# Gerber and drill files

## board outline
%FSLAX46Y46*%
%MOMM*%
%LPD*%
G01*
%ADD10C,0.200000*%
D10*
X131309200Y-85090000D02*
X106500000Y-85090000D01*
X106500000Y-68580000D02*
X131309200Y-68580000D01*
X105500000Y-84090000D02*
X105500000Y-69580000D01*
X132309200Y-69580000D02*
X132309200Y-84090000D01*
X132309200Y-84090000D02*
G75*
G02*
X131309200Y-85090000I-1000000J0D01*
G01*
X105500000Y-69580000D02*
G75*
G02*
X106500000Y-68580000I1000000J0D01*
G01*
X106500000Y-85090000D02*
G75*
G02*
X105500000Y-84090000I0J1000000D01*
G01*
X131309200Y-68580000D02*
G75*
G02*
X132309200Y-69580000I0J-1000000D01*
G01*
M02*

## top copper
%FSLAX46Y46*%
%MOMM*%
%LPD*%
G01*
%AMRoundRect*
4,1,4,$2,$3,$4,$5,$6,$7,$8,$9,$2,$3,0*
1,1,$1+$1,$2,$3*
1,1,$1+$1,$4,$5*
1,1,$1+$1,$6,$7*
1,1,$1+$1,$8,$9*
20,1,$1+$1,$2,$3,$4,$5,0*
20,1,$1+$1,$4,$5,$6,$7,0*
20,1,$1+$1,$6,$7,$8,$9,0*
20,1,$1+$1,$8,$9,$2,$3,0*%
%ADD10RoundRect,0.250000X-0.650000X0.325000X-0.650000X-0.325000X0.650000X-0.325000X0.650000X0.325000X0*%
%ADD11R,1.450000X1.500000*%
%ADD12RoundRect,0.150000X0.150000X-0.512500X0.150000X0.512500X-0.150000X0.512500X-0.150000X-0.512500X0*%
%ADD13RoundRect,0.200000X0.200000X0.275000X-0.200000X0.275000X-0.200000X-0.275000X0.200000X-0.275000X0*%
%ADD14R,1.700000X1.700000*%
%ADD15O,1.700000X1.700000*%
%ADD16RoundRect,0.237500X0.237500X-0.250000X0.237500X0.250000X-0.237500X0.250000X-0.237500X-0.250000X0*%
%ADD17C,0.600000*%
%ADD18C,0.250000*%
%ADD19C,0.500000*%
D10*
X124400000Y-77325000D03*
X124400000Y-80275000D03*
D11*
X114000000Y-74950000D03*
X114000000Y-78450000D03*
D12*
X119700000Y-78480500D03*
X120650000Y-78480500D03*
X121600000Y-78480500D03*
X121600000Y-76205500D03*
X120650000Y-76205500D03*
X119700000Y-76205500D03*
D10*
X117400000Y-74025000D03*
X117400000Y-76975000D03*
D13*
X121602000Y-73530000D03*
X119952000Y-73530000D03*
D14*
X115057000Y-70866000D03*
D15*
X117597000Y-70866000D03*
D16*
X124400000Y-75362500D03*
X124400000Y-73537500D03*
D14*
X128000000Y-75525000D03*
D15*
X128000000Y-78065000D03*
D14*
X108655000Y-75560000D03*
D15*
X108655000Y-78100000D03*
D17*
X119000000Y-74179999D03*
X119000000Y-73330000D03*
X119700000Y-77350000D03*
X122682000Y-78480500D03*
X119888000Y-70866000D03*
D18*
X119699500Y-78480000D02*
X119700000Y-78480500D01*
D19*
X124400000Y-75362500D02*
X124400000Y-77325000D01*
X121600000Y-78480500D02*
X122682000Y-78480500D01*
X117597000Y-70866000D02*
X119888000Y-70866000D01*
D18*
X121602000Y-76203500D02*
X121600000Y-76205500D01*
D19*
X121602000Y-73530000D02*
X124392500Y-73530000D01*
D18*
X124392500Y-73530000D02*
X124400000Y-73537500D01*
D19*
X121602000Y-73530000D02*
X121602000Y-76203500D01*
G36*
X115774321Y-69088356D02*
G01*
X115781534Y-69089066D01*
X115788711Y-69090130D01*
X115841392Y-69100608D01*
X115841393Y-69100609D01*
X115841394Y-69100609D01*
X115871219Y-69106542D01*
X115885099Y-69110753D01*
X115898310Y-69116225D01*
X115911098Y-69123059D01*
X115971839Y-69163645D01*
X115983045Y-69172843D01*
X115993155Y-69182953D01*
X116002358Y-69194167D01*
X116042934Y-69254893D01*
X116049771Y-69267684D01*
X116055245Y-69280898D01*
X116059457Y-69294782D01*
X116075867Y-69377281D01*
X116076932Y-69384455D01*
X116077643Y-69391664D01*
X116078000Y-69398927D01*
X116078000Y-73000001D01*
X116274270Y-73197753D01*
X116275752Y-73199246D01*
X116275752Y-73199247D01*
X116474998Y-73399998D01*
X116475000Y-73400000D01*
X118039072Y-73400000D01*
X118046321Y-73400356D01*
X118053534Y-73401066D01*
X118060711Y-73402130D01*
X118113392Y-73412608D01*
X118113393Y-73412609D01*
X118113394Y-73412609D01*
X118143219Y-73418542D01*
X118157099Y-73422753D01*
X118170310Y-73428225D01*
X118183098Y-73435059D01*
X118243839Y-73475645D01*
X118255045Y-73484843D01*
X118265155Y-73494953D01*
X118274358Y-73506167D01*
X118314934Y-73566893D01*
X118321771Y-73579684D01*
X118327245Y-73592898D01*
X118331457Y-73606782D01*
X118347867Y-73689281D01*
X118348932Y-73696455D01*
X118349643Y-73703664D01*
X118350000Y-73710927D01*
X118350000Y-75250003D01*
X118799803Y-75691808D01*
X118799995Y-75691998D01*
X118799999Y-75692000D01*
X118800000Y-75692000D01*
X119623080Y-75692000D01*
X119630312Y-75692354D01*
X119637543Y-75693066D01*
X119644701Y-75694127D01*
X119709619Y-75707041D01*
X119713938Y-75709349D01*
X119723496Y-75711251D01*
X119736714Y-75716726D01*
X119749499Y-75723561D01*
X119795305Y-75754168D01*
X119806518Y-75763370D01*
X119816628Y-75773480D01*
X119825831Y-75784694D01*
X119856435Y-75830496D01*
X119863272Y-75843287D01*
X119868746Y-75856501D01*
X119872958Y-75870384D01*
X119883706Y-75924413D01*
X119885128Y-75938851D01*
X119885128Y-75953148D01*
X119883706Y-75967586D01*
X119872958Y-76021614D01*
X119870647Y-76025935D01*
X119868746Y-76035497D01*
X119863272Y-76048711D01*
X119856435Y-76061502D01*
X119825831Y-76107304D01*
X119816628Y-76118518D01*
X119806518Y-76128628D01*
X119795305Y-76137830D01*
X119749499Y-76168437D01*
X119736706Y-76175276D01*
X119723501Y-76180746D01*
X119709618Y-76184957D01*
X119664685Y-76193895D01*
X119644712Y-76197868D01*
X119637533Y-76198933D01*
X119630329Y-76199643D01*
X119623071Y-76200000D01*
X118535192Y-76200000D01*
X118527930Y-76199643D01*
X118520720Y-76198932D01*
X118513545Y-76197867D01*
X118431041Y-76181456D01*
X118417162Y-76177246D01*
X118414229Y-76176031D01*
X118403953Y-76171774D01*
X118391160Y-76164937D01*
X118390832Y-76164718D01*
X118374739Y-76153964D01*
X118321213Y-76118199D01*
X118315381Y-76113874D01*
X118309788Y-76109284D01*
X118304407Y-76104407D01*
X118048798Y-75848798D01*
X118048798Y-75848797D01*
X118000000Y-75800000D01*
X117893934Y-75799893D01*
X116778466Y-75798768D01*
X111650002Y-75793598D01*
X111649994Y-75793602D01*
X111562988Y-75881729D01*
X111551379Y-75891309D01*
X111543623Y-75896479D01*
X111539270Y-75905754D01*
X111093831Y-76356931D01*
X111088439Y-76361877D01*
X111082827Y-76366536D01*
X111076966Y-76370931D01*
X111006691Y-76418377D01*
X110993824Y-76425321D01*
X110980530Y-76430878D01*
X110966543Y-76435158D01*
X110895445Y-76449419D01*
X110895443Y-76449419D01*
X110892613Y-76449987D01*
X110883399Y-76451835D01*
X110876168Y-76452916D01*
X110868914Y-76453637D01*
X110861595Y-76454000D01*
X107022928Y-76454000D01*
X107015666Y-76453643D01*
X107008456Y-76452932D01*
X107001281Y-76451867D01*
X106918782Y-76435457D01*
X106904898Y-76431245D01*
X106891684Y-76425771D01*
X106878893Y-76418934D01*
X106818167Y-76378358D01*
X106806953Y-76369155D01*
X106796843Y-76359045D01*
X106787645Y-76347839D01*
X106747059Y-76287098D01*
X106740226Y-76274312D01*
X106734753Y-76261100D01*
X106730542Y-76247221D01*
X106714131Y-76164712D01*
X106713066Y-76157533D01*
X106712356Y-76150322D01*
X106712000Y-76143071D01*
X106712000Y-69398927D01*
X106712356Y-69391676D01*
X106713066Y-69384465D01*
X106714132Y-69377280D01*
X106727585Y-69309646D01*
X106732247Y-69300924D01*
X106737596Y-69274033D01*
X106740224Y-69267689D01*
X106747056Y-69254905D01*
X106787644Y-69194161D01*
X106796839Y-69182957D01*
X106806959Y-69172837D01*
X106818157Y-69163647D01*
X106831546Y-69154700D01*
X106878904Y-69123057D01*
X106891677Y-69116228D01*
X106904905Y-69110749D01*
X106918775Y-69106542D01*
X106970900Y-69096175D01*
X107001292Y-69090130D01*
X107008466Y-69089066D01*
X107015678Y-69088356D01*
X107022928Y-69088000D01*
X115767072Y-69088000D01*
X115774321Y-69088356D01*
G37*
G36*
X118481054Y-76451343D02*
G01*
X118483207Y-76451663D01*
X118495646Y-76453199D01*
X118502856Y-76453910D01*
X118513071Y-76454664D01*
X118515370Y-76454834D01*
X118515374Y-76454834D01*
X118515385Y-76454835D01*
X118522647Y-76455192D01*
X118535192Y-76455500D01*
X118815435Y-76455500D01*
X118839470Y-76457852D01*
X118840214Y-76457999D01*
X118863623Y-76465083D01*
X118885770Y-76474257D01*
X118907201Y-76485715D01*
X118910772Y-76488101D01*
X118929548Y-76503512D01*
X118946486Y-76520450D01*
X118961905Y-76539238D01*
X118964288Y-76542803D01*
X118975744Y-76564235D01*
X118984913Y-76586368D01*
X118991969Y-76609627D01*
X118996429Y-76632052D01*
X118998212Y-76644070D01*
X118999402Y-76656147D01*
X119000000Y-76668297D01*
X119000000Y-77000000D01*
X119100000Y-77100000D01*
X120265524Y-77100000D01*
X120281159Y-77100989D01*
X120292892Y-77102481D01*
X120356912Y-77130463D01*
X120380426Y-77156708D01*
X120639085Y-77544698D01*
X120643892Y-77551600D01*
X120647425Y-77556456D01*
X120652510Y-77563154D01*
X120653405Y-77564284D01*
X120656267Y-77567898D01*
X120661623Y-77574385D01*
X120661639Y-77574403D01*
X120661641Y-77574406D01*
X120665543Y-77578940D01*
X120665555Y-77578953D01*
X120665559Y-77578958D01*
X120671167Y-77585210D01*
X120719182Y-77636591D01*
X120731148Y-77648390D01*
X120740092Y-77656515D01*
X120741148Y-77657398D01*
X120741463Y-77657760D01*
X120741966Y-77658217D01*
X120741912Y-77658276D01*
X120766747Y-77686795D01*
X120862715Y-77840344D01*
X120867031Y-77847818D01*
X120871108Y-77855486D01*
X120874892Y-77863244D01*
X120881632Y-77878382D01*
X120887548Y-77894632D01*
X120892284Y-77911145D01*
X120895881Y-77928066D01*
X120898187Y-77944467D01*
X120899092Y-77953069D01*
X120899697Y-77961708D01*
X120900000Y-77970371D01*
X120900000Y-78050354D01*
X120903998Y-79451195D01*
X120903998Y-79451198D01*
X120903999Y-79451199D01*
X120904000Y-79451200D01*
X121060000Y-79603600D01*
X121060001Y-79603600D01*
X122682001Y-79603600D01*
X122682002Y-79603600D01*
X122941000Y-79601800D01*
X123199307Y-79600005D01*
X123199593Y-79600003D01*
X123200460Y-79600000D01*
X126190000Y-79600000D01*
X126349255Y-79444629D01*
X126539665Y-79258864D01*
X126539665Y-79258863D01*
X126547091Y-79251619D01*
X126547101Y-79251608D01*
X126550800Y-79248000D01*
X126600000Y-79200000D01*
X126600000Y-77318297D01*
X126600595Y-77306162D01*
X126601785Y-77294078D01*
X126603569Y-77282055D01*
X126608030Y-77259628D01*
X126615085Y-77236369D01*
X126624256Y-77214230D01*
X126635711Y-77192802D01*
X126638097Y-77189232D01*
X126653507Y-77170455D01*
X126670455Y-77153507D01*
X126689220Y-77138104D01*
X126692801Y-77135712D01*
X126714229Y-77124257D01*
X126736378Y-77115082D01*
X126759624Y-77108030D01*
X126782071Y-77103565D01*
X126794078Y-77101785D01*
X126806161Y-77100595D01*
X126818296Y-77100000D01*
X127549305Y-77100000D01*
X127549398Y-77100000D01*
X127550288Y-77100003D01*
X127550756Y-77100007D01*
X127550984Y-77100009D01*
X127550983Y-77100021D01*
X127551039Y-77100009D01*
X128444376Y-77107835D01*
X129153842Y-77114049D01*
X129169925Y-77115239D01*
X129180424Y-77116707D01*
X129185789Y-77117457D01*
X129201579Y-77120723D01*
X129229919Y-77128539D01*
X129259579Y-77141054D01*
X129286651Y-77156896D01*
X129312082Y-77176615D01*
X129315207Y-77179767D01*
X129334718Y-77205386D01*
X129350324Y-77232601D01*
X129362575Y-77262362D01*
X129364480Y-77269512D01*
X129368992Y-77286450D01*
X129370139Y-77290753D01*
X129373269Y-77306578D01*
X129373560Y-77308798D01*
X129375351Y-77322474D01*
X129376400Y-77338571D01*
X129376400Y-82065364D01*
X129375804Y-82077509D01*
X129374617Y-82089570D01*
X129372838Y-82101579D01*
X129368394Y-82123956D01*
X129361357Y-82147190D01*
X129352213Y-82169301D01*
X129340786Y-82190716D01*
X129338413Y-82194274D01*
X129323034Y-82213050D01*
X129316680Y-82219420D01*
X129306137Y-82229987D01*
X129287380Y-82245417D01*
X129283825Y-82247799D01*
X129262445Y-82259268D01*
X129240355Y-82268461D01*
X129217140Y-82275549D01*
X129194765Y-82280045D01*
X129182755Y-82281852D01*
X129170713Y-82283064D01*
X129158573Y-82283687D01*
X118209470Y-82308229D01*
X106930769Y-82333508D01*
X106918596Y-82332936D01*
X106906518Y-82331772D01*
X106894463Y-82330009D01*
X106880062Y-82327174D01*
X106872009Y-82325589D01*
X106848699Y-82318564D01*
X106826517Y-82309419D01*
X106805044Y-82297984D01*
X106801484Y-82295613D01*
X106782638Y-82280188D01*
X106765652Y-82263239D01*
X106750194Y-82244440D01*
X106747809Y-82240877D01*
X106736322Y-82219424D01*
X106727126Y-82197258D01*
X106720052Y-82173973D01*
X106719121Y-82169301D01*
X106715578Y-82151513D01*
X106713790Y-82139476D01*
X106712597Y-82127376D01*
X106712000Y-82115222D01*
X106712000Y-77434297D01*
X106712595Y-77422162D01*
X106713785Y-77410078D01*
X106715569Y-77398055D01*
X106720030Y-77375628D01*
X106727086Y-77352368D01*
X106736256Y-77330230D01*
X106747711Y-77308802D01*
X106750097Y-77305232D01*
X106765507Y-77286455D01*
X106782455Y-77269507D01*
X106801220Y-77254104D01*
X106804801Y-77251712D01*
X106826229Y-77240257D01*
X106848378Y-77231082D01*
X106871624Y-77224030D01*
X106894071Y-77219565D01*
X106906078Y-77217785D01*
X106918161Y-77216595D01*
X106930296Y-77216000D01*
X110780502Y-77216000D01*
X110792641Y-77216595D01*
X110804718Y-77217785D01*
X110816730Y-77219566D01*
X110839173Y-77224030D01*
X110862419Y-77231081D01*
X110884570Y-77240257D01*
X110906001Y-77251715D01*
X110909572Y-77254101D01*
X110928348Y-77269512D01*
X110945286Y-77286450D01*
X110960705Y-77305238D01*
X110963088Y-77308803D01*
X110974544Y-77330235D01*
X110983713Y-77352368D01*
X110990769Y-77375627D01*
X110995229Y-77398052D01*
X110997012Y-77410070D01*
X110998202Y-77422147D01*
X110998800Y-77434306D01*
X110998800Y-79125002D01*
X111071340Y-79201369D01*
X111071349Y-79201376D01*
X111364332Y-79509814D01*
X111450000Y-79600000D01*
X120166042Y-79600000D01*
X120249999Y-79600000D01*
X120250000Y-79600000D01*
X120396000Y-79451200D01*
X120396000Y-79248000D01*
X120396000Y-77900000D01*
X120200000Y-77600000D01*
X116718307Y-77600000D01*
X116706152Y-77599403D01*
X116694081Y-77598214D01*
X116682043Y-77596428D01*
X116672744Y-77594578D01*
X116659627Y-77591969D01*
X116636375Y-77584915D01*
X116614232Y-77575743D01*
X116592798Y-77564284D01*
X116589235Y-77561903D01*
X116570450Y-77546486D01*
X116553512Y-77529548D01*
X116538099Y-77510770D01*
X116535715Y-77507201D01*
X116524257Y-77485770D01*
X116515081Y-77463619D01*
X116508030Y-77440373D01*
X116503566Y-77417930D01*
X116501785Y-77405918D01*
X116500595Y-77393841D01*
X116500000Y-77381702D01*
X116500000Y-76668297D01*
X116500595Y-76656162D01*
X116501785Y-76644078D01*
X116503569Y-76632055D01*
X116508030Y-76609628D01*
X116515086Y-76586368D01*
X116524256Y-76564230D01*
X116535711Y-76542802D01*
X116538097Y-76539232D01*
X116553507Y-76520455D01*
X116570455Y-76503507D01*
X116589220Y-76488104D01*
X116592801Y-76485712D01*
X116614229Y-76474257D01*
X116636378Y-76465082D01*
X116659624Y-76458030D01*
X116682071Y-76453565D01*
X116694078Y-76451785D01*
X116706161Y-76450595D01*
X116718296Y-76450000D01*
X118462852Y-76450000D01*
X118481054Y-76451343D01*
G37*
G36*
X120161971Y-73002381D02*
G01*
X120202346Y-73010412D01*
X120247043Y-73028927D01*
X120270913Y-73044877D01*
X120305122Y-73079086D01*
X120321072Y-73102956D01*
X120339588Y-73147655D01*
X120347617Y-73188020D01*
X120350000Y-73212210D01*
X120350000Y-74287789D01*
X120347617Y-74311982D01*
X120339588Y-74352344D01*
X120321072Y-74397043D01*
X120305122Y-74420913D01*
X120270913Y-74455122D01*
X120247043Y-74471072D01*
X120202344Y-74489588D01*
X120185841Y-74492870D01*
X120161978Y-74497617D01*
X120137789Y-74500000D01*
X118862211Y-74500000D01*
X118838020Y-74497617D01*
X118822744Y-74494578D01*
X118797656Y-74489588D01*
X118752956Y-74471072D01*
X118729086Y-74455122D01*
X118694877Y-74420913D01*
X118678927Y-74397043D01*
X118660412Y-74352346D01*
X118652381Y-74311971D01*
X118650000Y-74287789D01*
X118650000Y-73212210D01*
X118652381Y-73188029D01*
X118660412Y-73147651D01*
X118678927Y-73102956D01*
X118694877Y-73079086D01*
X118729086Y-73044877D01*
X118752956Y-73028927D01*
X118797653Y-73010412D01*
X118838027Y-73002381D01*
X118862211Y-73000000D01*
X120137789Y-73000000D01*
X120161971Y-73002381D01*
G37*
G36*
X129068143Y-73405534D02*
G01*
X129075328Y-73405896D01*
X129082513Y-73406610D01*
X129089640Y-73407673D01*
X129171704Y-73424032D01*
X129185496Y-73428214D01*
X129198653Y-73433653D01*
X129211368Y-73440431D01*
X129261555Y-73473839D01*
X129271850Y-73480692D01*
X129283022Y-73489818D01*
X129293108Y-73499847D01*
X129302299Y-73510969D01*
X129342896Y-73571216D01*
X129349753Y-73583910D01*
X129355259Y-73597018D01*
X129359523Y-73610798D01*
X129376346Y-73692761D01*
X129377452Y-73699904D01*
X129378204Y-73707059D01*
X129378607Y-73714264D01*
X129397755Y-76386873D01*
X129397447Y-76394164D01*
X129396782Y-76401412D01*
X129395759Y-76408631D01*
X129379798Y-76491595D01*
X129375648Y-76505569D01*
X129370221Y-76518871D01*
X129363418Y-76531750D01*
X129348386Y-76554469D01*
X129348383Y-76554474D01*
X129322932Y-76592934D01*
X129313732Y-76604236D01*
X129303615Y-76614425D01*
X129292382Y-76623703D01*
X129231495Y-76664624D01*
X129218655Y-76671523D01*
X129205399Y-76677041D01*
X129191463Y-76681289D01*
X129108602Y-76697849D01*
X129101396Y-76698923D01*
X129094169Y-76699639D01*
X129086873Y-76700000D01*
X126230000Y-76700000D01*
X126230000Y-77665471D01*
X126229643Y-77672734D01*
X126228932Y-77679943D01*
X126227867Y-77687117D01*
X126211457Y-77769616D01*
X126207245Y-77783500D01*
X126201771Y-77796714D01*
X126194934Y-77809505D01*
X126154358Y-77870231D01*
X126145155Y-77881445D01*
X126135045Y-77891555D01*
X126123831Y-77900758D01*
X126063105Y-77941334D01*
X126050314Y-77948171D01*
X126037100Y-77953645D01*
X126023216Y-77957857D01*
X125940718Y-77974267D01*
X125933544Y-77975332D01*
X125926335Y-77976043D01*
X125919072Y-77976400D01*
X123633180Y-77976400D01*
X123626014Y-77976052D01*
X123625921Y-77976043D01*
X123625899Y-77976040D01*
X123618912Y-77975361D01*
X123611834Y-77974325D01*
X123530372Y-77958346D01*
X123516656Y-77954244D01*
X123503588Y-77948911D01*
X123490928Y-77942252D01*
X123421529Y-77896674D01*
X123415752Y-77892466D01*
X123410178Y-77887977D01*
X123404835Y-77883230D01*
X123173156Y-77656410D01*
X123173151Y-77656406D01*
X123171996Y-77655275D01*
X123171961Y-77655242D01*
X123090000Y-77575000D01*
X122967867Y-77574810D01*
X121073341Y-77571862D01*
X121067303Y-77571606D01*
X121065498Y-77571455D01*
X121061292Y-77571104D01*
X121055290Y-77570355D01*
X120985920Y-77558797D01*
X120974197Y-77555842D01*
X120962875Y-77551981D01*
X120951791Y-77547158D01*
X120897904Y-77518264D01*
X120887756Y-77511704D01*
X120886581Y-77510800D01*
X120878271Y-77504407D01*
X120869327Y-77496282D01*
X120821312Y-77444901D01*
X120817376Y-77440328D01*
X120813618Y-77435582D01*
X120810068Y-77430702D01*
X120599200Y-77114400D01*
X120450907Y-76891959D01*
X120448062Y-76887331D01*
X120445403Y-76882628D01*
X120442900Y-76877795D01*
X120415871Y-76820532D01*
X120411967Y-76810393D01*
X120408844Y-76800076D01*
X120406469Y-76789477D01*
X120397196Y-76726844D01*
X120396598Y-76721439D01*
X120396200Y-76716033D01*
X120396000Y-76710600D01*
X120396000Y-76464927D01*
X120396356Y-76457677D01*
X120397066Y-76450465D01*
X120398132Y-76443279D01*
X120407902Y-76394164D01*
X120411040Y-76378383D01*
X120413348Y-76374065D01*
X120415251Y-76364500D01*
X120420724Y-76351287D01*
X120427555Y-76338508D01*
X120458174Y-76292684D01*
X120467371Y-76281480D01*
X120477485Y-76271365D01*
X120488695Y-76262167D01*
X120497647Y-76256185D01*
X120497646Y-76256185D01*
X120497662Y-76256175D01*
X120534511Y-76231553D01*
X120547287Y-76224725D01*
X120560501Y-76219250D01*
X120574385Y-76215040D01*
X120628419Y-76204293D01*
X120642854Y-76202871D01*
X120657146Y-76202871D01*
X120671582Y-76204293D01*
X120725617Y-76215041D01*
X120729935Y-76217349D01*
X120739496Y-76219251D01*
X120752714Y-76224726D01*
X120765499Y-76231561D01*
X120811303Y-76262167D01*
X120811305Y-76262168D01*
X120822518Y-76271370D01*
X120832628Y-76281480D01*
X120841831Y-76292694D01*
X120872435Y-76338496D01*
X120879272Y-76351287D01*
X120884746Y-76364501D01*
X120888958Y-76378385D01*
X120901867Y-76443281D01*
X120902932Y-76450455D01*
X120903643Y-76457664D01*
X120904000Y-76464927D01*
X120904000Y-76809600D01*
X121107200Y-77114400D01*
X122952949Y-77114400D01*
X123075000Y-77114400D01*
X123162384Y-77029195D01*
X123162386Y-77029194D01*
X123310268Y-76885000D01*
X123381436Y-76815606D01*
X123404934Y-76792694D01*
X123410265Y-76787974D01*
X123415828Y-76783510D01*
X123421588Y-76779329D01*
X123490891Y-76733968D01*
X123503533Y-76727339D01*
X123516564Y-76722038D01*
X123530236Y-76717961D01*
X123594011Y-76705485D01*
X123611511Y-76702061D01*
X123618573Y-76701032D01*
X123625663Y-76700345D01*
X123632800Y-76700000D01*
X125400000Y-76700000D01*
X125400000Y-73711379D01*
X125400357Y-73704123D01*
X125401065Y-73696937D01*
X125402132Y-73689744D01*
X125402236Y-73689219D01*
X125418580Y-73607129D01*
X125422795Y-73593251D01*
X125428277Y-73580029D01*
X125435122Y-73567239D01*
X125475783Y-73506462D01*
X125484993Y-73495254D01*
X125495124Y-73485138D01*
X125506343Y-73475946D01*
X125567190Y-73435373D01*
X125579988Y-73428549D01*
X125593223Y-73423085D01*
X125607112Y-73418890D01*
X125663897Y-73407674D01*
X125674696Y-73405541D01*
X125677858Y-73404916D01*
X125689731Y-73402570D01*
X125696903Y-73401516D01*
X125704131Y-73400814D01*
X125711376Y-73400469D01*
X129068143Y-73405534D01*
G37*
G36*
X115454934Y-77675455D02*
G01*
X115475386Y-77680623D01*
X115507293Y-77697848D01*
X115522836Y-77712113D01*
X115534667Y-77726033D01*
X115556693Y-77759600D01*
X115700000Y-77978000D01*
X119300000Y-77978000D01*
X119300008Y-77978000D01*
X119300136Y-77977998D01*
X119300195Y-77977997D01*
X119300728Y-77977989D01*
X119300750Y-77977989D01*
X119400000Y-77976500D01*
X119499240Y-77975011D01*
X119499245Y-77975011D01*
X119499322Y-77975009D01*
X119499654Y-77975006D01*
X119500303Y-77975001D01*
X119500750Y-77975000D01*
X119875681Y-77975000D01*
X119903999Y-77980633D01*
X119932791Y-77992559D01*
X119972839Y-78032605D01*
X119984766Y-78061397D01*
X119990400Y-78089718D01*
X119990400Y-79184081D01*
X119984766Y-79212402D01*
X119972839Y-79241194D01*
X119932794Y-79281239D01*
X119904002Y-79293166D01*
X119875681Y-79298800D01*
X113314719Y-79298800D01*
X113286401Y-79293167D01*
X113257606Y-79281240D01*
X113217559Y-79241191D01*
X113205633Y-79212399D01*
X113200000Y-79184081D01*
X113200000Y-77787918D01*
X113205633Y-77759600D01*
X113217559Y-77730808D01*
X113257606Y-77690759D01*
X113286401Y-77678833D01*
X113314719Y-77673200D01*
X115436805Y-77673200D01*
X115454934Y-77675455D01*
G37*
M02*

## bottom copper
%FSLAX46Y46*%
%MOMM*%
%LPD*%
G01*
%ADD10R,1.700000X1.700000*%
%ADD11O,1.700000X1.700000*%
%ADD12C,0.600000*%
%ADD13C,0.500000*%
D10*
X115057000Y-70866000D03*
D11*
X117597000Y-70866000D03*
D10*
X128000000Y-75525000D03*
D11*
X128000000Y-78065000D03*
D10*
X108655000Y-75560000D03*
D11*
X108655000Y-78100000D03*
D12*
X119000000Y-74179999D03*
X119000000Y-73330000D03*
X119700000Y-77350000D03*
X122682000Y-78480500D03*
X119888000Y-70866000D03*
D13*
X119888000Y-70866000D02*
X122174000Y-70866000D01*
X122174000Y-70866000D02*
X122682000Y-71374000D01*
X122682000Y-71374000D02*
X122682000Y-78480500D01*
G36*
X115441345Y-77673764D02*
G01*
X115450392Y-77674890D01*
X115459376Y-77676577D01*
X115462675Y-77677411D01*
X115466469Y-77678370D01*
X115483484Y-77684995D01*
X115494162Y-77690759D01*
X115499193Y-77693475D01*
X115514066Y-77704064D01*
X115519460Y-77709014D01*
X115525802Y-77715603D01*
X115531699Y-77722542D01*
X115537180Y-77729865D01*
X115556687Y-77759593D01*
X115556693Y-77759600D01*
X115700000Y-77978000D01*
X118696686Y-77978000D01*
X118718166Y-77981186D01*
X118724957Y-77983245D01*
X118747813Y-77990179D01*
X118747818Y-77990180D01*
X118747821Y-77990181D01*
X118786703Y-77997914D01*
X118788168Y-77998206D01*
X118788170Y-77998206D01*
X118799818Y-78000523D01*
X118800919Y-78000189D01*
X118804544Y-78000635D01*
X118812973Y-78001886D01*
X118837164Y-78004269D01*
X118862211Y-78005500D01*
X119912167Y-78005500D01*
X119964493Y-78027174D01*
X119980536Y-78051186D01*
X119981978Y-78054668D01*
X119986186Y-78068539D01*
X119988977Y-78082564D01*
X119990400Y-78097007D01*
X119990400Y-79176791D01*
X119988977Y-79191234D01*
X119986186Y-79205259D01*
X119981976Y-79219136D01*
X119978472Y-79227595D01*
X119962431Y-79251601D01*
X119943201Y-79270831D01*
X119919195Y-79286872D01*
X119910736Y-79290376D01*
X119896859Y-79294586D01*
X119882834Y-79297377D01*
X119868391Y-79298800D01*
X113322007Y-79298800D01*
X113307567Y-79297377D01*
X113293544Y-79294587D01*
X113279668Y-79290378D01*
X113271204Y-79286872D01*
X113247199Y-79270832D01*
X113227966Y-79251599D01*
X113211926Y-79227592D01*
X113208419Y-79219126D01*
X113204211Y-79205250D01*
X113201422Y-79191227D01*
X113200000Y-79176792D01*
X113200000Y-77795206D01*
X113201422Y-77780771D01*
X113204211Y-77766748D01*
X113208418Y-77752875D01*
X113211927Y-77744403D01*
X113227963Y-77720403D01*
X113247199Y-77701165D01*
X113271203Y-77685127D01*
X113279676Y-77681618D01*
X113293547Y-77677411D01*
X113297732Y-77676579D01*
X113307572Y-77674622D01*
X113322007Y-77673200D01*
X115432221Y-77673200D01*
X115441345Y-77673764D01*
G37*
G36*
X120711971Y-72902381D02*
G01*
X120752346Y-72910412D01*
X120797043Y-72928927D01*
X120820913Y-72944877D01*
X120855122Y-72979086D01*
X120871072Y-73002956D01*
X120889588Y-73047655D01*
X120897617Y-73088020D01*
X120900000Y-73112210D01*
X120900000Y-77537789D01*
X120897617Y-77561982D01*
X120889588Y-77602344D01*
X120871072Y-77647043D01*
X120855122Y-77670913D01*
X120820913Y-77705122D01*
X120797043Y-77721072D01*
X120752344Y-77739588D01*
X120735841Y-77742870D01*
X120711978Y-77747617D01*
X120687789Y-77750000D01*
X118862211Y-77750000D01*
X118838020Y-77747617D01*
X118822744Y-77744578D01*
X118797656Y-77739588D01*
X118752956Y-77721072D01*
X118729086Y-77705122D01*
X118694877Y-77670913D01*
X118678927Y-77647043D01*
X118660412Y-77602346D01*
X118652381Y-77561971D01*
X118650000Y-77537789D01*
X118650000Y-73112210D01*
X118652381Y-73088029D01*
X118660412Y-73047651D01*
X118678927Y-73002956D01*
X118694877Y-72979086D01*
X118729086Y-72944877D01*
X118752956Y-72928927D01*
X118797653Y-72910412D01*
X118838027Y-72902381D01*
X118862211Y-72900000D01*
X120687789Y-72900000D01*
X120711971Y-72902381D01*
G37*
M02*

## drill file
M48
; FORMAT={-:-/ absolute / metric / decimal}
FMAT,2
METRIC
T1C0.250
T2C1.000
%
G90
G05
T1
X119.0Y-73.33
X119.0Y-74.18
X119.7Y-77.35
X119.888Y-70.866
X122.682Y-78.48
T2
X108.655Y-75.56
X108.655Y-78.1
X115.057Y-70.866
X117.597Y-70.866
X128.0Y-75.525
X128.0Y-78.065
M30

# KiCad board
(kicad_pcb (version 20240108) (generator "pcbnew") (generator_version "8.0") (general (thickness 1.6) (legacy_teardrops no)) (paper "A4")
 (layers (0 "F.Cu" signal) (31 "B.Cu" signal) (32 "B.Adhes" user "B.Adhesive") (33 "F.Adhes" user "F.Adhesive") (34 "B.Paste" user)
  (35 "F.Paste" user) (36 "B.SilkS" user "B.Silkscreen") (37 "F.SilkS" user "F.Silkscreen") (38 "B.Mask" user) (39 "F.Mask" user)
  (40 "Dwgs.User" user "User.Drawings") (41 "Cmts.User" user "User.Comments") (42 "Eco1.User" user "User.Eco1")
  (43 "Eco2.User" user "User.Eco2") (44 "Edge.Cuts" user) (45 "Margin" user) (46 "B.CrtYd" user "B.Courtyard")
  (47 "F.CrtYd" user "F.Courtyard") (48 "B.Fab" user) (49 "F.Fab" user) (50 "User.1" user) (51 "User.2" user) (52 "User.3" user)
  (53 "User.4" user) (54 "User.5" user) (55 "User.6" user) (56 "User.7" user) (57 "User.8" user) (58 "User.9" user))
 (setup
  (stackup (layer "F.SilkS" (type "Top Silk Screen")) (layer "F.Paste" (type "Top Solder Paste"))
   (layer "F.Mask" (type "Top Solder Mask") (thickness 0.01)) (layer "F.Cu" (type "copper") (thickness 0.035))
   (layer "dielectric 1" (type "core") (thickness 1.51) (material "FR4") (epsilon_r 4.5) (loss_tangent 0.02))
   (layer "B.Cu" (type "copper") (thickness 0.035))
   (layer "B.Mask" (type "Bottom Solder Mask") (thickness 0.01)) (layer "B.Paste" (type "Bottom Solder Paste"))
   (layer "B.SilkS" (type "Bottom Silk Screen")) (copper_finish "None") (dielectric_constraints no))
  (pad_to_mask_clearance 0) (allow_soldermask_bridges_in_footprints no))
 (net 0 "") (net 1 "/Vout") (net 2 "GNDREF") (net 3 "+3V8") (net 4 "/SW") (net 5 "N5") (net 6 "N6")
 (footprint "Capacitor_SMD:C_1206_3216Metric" (layer "F.Cu") (at 124.4 78.8 -90)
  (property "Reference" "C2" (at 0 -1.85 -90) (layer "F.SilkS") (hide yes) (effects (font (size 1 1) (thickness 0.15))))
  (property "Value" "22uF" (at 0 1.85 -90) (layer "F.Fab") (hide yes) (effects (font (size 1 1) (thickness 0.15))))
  (pad "1" smd roundrect (at -1.475 0 270) (size 1.15 1.8) (layers "F.Cu" "F.Paste" "F.Mask") (roundrect_rratio 0.217391) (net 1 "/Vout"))
  (pad "2" smd roundrect (at 1.475 0 270) (size 1.15 1.8) (layers "F.Cu" "F.Paste" "F.Mask") (roundrect_rratio 0.217391) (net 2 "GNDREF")))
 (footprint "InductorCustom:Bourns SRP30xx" (layer "F.Cu") (at 114 76.7 -90)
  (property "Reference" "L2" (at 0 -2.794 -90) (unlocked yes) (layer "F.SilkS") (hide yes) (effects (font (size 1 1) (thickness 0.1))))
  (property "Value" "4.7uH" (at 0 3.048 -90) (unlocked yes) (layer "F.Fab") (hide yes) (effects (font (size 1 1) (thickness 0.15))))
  (pad "1" smd rect (at -1.75 0 270) (size 1.5 1.45) (layers "F.Cu" "F.Paste" "F.Mask") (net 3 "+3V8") (thermal_bridge_angle 45))
  (pad "2" smd rect (at 1.75 0 270) (size 1.5 1.45) (layers "F.Cu" "F.Paste" "F.Mask") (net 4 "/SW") (thermal_bridge_angle 45)))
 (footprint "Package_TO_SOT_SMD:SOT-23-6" (layer "F.Cu") (at 120.65 77.343 90)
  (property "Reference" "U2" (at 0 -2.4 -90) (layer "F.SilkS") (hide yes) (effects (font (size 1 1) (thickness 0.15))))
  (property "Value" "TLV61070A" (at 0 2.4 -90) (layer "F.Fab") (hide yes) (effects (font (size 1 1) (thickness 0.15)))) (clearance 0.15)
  (pad "1" smd roundrect (at -1.1375 -0.95 90) (size 1.325 0.6) (layers "F.Cu" "F.Paste" "F.Mask") (roundrect_rratio 0.25) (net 4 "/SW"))
  (pad "2" smd roundrect (at -1.1375 0 90) (size 1.325 0.6) (layers "F.Cu" "F.Paste" "F.Mask") (roundrect_rratio 0.25) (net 2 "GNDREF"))
  (pad "3" smd roundrect (at -1.1375 0.95 90) (size 1.325 0.6) (layers "F.Cu" "F.Paste" "F.Mask") (roundrect_rratio 0.25) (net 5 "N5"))
  (pad "4" smd roundrect (at 1.1375 0.95 90) (size 1.325 0.6) (layers "F.Cu" "F.Paste" "F.Mask") (roundrect_rratio 0.25) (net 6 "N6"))
  (pad "5" smd roundrect (at 1.1375 0 90) (size 1.325 0.6) (layers "F.Cu" "F.Paste" "F.Mask") (roundrect_rratio 0.25) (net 1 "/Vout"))
  (pad "6" smd roundrect (at 1.1375 -0.95 90) (size 1.325 0.6) (layers "F.Cu" "F.Paste" "F.Mask") (roundrect_rratio 0.25) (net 3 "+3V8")))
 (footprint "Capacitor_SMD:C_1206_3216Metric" (layer "F.Cu") (at 117.4 75.5 -90)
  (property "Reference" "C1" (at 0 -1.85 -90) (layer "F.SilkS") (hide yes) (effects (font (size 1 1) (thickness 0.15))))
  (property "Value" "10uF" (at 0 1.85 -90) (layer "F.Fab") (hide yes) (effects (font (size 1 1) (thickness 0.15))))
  (pad "1" smd roundrect (at -1.475 0 270) (size 1.15 1.8) (layers "F.Cu" "F.Paste" "F.Mask") (roundrect_rratio 0.217391) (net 3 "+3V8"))
  (pad "2" smd roundrect (at 1.475 0 270) (size 1.15 1.8) (layers "F.Cu" "F.Paste" "F.Mask") (roundrect_rratio 0.217391) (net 2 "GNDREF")))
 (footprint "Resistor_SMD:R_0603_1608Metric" (layer "F.Cu") (at 120.777 73.53 180)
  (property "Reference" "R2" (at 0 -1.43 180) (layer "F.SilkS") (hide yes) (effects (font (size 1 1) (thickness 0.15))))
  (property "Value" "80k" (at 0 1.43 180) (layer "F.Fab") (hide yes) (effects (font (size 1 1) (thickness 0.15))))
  (pad "1" smd roundrect (at -0.825 0 180) (size 0.8 0.95) (layers "F.Cu" "F.Paste" "F.Mask") (roundrect_rratio 0.25) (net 6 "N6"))
  (pad "2" smd roundrect (at 0.825 0 180) (size 0.8 0.95) (layers "F.Cu" "F.Paste" "F.Mask") (roundrect_rratio 0.25) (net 2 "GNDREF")))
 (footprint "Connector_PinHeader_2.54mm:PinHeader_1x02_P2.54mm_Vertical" (layer "F.Cu") (at 115.057 70.866 90)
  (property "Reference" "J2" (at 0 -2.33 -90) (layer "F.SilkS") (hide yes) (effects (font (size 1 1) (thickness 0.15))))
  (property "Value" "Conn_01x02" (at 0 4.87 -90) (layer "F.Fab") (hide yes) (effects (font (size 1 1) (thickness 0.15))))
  (pad "1" thru_hole rect (at 0 0 90) (size 1.7 1.7) (drill 1) (layers "*.Cu" "*.Mask") (remove_unused_layers no) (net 3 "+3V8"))
  (pad "2" thru_hole oval (at 0 2.54 90) (size 1.7 1.7) (drill 1) (layers "*.Cu" "*.Mask") (remove_unused_layers no) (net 5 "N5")))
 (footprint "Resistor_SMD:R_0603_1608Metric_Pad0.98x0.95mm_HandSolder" (layer "F.Cu") (at 124.4 74.45 90)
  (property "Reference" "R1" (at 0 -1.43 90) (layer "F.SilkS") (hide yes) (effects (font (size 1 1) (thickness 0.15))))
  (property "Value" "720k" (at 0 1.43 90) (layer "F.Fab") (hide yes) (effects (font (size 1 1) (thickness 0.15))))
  (pad "1" smd roundrect (at -0.9125 0 90) (size 0.975 0.95) (layers "F.Cu" "F.Paste" "F.Mask") (roundrect_rratio 0.25) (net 1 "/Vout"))
  (pad "2" smd roundrect (at 0.9125 0 90) (size 0.975 0.95) (layers "F.Cu" "F.Paste" "F.Mask") (roundrect_rratio 0.25) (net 6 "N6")))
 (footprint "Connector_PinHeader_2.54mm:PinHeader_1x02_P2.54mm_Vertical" (layer "B.Cu") (at 128 75.525 180)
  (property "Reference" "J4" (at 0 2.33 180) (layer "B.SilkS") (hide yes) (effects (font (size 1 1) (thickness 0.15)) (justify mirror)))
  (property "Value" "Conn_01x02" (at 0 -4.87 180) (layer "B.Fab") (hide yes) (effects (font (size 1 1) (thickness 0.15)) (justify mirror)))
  (pad "1" thru_hole rect (at 0 0 180) (size 1.7 1.7) (drill 1) (layers "*.Cu" "*.Mask") (remove_unused_layers no) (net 1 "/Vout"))
  (pad "2" thru_hole oval (at 0 -2.54 180) (size 1.7 1.7) (drill 1) (layers "*.Cu" "*.Mask") (remove_unused_layers no) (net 2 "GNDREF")))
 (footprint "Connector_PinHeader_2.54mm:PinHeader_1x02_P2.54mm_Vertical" (layer "B.Cu") (at 108.655 75.56 180)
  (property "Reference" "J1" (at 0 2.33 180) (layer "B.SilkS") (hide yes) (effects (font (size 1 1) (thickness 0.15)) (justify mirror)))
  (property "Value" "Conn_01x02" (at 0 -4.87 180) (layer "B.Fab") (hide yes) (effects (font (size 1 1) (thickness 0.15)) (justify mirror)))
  (pad "1" thru_hole rect (at 0 0 180) (size 1.7 1.7) (drill 1) (layers "*.Cu" "*.Mask") (remove_unused_layers no) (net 3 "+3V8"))
  (pad "2" thru_hole oval (at 0 -2.54 180) (size 1.7 1.7) (drill 1) (layers "*.Cu" "*.Mask") (remove_unused_layers no) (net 2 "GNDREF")))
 (gr_line (start 131.3092 85.09) (end 106.5 85.09) (stroke (width 0.2) (type default)) (layer "Edge.Cuts"))
 (gr_line (start 106.5 68.58) (end 131.3092 68.58) (stroke (width 0.2) (type default)) (layer "Edge.Cuts"))
 (gr_line (start 105.5 84.09) (end 105.5 69.58) (stroke (width 0.2) (type default)) (layer "Edge.Cuts"))
 (gr_line (start 132.3092 69.58) (end 132.3092 84.09) (stroke (width 0.2) (type default)) (layer "Edge.Cuts"))
 (gr_arc (start 132.3092 84.09) (mid 132.016307 84.797107) (end 131.3092 85.09) (stroke (width 0.2) (type default)) (layer "Edge.Cuts"))
 (gr_arc (start 105.5 69.58) (mid 105.792893 68.872893) (end 106.5 68.58) (stroke (width 0.2) (type default)) (layer "Edge.Cuts"))
 (gr_arc (start 106.5 85.09) (mid 105.792893 84.797107) (end 105.5 84.09) (stroke (width 0.2) (type default)) (layer "Edge.Cuts"))
 (gr_arc (start 131.3092 68.58) (mid 132.016307 68.872893) (end 132.3092 69.58) (stroke (width 0.2) (type default)) (layer "Edge.Cuts"))
 (via (at 119 74.179999) (size 0.6) (drill 0.25) (layers "F.Cu" "B.Cu") (free yes) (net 2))
 (via (at 119 73.33) (size 0.6) (drill 0.25) (layers "F.Cu" "B.Cu") (free yes) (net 2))
 (via (at 119.7 77.35) (size 0.6) (drill 0.25) (layers "F.Cu" "B.Cu") (free yes) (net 2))
 (segment (start 119.6995 78.48) (end 119.7 78.4805) (width 0.25) (layer "F.Cu") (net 4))
 (segment (start 124.4 75.3625) (end 124.4 77.325) (width 0.5) (layer "F.Cu") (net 1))
 (segment (start 121.6 78.4805) (end 122.682 78.4805) (width 0.5) (layer "F.Cu") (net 5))
 (segment (start 117.597 70.866) (end 119.888 70.866) (width 0.5) (layer "F.Cu") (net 5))
 (via (at 122.682 78.4805) (size 0.6) (drill 0.25) (layers "F.Cu" "B.Cu") (free yes) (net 5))
 (via (at 119.888 70.866) (size 0.6) (drill 0.25) (layers "F.Cu" "B.Cu") (free yes) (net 5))
 (segment (start 119.888 70.866) (end 122.174 70.866) (width 0.5) (layer "B.Cu") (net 5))
 (segment (start 122.174 70.866) (end 122.682 71.374) (width 0.5) (layer "B.Cu") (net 5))
 (segment (start 122.682 71.374) (end 122.682 78.4805) (width 0.5) (layer "B.Cu") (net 5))
 (segment (start 121.602 76.2035) (end 121.6 76.2055) (width 0.25) (layer "F.Cu") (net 6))
 (segment (start 121.602 73.53) (end 124.3925 73.53) (width 0.5) (layer "F.Cu") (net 6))
 (segment (start 124.3925 73.53) (end 124.4 73.5375) (width 0.25) (layer "F.Cu") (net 6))
 (segment (start 121.602 73.53) (end 121.602 76.2035) (width 0.5) (layer "F.Cu") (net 6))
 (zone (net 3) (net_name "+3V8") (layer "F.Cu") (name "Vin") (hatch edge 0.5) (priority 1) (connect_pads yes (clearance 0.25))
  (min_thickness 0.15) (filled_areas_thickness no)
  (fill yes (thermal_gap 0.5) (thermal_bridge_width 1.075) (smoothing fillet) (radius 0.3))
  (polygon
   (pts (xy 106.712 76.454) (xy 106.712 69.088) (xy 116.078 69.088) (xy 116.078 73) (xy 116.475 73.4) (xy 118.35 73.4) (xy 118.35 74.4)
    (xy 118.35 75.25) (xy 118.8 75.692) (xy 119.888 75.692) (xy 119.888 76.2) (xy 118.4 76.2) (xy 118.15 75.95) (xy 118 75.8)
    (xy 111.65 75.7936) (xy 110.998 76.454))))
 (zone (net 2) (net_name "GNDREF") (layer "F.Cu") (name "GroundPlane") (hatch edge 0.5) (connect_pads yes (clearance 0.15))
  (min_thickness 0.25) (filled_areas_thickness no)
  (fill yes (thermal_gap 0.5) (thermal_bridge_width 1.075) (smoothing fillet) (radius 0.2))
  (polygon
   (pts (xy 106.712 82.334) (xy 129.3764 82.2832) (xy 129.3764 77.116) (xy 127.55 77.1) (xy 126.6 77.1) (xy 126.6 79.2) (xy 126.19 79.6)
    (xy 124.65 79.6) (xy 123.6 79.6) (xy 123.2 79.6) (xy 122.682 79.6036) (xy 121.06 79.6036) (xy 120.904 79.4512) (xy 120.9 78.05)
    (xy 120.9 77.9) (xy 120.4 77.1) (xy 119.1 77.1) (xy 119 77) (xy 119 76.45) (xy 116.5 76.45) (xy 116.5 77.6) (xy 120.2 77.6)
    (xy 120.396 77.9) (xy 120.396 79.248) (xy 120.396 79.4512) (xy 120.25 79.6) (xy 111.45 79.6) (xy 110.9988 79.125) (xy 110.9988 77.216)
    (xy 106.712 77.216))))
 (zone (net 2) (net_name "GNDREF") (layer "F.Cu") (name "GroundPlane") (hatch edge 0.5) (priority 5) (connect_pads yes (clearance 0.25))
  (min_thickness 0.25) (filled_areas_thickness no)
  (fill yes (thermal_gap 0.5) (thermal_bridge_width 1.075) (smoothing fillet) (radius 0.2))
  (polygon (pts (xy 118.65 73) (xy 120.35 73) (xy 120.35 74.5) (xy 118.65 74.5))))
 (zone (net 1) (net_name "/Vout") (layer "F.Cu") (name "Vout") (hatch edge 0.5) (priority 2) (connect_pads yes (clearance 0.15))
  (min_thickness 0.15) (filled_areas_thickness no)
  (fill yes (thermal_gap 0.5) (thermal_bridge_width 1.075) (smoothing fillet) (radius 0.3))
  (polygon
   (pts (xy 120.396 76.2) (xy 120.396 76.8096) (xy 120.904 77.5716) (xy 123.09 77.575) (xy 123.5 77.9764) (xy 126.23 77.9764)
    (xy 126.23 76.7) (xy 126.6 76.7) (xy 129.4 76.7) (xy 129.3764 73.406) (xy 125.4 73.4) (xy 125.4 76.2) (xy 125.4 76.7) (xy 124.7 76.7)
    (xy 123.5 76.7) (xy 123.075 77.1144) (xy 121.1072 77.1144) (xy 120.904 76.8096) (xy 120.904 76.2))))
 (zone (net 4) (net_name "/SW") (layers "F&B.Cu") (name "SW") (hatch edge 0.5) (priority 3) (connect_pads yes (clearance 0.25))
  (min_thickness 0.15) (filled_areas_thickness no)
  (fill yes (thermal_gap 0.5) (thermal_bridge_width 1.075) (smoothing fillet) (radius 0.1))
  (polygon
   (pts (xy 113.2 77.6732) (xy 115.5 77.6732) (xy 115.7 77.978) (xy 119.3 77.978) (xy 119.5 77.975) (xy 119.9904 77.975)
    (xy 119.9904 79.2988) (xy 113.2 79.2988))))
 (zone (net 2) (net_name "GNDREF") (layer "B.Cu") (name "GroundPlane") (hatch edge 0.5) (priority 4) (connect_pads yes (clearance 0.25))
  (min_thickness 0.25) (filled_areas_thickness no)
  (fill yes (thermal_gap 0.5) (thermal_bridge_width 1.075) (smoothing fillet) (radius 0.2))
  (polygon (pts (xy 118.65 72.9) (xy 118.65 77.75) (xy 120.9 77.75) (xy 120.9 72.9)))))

